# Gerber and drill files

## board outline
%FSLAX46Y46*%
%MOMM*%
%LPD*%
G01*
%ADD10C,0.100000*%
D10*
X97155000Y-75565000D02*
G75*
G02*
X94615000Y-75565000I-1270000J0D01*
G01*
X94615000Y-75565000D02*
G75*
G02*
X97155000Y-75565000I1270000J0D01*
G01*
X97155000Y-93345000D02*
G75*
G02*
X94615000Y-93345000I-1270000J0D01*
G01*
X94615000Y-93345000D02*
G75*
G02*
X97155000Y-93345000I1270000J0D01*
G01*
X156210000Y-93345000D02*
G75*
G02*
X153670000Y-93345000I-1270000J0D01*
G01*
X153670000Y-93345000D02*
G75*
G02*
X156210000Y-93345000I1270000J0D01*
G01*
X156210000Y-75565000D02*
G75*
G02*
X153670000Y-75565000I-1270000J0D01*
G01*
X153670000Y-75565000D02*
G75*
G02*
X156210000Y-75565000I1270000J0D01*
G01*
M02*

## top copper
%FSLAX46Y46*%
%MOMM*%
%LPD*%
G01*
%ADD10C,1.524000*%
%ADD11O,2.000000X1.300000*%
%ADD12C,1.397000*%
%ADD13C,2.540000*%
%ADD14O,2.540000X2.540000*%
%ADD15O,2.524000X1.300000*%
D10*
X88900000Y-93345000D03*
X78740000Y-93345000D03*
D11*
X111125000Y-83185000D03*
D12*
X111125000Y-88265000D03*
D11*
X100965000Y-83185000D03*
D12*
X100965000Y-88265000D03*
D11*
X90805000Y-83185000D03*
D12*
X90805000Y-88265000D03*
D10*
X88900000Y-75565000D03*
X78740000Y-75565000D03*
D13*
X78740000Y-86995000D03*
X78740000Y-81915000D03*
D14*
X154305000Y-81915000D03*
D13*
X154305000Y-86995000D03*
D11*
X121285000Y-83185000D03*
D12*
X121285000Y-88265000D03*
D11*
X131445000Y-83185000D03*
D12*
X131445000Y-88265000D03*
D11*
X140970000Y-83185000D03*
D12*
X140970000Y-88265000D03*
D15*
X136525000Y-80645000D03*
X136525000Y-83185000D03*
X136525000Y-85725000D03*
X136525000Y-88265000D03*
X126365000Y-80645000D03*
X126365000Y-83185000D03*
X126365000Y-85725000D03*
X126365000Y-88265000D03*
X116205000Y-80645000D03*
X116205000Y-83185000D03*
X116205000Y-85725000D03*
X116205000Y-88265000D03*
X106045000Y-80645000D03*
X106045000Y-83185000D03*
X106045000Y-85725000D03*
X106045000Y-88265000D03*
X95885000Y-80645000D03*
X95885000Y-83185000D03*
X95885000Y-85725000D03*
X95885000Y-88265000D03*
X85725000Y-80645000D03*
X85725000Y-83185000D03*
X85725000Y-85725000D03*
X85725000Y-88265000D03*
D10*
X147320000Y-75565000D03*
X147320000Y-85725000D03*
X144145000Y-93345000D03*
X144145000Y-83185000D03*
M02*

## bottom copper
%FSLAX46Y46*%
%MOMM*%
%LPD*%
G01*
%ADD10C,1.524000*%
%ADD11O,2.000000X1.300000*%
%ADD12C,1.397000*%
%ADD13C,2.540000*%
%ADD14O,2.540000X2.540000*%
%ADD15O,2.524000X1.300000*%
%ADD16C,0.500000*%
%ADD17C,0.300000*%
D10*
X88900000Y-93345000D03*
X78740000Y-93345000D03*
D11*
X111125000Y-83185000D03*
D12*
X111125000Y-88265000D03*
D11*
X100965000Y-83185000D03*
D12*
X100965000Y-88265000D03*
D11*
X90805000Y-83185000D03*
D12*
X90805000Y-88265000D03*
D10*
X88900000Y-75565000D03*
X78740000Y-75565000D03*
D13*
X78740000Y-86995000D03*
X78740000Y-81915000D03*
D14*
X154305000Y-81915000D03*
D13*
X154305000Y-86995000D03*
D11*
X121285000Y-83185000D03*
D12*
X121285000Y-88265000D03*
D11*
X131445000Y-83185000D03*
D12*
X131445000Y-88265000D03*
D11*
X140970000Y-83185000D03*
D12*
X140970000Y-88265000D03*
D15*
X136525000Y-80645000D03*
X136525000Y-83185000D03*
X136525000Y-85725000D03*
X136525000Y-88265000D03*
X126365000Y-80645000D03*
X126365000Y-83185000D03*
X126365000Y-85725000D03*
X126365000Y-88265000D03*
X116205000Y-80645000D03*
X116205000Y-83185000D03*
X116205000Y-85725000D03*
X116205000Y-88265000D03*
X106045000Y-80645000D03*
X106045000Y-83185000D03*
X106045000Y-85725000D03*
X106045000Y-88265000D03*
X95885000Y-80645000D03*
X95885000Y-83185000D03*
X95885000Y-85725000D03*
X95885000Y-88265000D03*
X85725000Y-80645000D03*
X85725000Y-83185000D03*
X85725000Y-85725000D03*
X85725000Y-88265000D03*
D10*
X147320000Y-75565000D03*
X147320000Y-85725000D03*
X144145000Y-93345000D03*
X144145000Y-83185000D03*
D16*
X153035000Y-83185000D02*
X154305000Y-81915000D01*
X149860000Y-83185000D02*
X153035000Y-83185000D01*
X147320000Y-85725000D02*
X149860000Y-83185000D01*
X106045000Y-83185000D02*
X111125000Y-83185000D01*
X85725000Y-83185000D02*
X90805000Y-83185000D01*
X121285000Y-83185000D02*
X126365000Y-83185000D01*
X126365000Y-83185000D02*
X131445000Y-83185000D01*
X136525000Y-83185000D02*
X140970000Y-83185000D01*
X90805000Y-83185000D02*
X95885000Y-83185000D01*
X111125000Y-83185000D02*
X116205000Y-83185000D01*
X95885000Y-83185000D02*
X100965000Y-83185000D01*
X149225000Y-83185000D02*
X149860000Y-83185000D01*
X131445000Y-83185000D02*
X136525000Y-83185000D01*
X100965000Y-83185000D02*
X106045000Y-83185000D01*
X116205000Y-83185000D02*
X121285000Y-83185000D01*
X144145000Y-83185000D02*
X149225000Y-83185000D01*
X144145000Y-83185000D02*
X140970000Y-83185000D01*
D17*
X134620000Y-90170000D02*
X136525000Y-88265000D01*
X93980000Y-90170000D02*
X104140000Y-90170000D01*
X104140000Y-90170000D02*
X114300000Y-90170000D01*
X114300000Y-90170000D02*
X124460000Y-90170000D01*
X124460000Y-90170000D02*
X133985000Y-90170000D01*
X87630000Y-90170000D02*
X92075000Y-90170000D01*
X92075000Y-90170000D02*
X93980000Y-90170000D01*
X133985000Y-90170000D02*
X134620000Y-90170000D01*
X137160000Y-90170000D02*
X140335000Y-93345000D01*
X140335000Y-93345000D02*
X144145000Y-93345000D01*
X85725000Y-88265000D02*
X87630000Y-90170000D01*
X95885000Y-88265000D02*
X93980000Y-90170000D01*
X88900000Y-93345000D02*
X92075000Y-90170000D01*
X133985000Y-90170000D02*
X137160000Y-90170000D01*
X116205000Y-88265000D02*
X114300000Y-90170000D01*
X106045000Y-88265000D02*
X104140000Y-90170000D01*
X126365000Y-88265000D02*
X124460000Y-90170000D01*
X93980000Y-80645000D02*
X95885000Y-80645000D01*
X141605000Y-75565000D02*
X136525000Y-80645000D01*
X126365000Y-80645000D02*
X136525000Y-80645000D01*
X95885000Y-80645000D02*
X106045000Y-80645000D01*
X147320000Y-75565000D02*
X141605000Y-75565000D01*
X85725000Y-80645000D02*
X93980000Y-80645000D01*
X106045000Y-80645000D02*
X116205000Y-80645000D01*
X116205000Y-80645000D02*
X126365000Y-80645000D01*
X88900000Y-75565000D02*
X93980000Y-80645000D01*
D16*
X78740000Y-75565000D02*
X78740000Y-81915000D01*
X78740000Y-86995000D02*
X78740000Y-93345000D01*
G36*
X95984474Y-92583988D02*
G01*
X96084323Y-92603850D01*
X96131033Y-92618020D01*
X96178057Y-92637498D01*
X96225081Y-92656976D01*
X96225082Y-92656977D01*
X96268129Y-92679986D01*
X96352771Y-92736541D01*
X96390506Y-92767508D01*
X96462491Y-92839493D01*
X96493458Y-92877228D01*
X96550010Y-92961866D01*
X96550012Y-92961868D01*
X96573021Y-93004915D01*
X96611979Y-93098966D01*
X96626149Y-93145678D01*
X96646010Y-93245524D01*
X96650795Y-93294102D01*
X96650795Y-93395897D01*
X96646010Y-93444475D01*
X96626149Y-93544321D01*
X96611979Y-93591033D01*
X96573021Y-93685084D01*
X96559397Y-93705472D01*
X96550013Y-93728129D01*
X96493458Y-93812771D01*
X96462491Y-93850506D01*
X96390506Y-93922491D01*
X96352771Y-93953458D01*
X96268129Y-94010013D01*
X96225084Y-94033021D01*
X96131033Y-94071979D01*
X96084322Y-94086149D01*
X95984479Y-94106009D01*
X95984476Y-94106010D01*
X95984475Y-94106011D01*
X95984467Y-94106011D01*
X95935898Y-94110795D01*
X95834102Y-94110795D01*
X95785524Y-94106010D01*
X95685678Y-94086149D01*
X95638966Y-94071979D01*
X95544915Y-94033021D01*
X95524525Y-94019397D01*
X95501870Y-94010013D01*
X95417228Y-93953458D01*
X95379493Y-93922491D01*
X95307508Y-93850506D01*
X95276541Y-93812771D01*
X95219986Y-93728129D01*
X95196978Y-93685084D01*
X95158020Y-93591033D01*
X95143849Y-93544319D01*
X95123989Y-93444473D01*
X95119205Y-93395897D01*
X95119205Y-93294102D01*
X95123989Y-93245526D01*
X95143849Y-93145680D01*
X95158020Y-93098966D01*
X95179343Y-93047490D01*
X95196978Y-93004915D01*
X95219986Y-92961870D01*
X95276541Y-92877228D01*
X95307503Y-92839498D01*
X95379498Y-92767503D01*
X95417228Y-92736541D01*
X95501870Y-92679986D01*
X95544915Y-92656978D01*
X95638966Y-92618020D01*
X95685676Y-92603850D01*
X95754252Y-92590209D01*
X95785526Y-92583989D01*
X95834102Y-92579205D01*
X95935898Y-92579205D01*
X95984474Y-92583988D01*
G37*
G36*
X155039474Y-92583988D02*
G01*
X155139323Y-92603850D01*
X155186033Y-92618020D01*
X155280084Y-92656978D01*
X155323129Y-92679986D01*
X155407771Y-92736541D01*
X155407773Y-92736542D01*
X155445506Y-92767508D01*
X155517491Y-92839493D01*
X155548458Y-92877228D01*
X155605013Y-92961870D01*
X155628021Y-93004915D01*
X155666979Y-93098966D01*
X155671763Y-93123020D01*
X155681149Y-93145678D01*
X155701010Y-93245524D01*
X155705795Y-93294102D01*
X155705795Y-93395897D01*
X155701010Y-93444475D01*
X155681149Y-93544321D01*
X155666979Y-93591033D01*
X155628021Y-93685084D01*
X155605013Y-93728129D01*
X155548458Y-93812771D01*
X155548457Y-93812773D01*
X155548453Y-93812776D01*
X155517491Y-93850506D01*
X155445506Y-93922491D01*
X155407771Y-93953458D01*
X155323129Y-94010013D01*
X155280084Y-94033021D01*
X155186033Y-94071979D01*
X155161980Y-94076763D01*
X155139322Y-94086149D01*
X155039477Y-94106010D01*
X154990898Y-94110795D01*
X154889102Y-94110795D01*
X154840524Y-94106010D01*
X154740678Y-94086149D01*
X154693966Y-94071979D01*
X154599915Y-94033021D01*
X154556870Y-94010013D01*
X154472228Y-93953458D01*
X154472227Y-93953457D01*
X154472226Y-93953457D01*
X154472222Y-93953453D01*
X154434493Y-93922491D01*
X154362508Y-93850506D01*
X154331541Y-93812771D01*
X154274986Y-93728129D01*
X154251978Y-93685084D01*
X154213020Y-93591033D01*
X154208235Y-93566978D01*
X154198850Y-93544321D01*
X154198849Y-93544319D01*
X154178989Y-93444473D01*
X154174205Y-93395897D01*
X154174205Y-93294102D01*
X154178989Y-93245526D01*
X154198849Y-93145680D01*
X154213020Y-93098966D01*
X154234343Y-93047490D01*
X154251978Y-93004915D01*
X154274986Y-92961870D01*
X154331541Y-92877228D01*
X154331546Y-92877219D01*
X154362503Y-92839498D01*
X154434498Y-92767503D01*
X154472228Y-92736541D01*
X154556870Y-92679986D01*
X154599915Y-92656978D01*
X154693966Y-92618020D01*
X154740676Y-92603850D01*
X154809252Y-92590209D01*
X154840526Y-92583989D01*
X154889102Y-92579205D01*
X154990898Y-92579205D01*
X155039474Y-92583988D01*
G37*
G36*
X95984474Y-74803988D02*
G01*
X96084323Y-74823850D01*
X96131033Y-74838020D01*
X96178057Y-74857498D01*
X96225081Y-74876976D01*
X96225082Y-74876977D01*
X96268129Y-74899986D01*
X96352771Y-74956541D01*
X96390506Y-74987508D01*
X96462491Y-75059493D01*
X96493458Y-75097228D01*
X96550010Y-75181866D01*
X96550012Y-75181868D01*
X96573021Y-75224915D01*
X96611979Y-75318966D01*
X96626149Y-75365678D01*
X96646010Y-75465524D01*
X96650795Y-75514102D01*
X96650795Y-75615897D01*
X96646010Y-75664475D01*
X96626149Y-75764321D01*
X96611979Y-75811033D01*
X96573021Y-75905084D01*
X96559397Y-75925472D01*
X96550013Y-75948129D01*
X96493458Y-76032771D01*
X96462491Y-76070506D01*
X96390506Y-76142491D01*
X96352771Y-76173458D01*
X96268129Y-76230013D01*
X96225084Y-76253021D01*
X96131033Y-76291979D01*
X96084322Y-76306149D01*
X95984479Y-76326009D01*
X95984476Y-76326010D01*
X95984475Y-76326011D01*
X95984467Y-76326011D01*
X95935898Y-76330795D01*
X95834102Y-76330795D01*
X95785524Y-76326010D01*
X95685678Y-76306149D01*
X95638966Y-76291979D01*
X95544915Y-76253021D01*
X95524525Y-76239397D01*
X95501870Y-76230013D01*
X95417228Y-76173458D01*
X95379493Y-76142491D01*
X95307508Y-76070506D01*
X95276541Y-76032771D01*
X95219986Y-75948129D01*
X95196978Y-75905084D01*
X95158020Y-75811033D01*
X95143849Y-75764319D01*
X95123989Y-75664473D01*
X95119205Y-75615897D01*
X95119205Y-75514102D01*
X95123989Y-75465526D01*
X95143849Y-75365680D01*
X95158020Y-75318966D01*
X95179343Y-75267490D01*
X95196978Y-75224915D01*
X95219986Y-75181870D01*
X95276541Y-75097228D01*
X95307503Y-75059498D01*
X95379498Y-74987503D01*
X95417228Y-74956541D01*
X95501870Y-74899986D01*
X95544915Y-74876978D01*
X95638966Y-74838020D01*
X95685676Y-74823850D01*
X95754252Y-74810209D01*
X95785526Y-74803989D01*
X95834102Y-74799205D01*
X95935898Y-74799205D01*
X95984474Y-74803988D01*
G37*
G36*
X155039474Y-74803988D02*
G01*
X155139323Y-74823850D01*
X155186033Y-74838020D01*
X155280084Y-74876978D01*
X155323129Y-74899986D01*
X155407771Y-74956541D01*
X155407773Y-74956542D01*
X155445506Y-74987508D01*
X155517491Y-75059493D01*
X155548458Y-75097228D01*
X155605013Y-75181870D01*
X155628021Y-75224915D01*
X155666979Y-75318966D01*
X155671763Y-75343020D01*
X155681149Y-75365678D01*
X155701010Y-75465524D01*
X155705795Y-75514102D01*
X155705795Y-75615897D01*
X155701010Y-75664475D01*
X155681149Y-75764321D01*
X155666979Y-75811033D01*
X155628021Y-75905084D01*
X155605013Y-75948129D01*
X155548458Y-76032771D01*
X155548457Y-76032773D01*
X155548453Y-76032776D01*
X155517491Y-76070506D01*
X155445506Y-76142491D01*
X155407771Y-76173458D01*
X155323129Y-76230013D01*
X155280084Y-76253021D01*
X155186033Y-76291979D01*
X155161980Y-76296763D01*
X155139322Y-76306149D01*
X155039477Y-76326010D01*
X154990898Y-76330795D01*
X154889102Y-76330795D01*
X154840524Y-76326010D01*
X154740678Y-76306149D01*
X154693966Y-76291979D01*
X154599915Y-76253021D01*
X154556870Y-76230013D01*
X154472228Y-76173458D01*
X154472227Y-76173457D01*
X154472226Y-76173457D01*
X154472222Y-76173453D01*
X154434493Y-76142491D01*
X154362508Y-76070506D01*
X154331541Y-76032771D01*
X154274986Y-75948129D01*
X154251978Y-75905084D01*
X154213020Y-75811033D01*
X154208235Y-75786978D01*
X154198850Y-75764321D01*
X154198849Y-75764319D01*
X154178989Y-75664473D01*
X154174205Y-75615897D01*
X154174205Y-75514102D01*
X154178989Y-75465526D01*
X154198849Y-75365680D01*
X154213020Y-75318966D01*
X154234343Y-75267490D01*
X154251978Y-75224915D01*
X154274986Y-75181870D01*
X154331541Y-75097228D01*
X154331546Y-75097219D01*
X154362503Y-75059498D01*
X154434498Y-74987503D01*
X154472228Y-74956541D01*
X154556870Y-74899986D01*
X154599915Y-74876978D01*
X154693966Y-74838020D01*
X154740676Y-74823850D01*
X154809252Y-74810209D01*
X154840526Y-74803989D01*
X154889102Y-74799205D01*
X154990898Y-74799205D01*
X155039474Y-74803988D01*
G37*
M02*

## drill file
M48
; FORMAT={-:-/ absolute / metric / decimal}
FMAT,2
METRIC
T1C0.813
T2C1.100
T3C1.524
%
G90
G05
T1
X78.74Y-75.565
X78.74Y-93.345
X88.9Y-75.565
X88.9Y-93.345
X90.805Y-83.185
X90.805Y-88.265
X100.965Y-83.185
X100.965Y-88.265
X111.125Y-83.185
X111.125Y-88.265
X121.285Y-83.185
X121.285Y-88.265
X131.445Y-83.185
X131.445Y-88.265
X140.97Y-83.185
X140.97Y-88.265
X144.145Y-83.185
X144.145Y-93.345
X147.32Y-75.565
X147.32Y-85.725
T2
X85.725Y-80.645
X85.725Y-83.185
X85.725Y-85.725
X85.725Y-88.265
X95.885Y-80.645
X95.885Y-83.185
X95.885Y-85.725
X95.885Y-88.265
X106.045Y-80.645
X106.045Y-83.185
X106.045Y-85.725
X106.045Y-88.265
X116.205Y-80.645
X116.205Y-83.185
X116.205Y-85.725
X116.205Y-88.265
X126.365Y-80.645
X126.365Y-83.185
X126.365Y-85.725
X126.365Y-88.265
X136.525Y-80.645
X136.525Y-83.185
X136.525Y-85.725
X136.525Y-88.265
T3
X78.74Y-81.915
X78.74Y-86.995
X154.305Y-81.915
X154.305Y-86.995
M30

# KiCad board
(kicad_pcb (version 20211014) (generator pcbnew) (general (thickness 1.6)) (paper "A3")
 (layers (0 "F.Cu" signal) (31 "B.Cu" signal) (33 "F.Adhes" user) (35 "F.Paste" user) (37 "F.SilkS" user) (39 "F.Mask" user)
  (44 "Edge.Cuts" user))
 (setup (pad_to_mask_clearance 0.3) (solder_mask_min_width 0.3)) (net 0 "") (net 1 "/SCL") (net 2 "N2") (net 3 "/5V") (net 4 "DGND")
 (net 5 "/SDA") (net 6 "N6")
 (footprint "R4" (layer "F.Cu") (at 83.82 93.345 180) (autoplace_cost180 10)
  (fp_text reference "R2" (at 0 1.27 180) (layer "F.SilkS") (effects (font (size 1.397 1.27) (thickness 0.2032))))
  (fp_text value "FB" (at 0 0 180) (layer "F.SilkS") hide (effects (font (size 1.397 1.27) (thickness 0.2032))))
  (pad "1" thru_hole circle locked (at -5.08 0 180) (size 1.524 1.524) (drill 0.8128) (layers *.Cu *.Mask "F.SilkS") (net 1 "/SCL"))
  (pad "2" thru_hole circle locked (at 5.08 0 180) (size 1.524 1.524) (drill 0.8128) (layers *.Cu *.Mask "F.SilkS") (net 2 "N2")))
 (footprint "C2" (layer "F.Cu") (at 111.125 85.725 -90)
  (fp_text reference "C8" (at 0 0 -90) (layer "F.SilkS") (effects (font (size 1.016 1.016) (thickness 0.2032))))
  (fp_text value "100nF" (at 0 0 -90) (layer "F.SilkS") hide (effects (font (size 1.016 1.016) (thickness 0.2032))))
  (pad "1" thru_hole oval locked (at -2.54 0 270) (size 1.3 2) (drill 0.8128) (layers *.Cu *.Mask "F.SilkS") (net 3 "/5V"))
  (pad "2" thru_hole circle locked (at 2.54 0 270) (size 1.397 1.397) (drill 0.8128) (layers *.Cu *.Mask "F.SilkS") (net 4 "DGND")))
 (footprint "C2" (layer "F.Cu") (at 100.965 85.725 -90)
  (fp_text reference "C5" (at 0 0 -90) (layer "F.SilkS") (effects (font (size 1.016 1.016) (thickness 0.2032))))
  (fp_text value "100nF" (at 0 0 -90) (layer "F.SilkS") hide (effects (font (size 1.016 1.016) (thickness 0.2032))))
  (pad "1" thru_hole oval locked (at -2.54 0 270) (size 1.3 2) (drill 0.8128) (layers *.Cu *.Mask "F.SilkS") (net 3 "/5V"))
  (pad "2" thru_hole circle locked (at 2.54 0 270) (size 1.397 1.397) (drill 0.8128) (layers *.Cu *.Mask "F.SilkS") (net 4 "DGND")))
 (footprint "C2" (layer "F.Cu") (at 90.805 85.725 -90)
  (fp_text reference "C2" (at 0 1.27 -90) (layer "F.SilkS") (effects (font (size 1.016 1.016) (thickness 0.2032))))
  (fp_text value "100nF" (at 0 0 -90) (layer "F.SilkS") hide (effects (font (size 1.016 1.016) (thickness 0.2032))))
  (pad "1" thru_hole oval locked (at -2.54 0 270) (size 1.3 2) (drill 0.8128) (layers *.Cu *.Mask "F.SilkS") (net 3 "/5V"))
  (pad "2" thru_hole circle locked (at 2.54 0 270) (size 1.397 1.397) (drill 0.8128) (layers *.Cu *.Mask "F.SilkS") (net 4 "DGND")))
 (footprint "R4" (layer "F.Cu") (at 83.82 75.565 180) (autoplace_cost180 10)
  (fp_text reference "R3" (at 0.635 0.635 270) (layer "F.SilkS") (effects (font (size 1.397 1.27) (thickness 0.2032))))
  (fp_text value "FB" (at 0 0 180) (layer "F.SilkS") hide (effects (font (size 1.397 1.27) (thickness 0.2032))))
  (pad "1" thru_hole circle locked (at -5.08 0 180) (size 1.524 1.524) (drill 0.8128) (layers *.Cu *.Mask "F.SilkS") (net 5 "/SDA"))
  (pad "2" thru_hole circle locked (at 5.08 0 180) (size 1.524 1.524) (drill 0.8128) (layers *.Cu *.Mask "F.SilkS") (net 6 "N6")))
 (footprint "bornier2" (layer "F.Cu") (at 78.74 84.455 90)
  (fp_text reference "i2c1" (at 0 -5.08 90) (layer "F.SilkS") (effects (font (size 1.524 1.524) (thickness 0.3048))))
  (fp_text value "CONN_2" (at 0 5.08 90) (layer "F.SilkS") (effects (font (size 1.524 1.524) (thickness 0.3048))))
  (pad "1" thru_hole circle locked (at -2.54 0 90) (size 2.54 2.54) (drill 1.524) (layers *.Cu *.Mask "F.SilkS") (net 2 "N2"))
  (pad "2" thru_hole circle locked (at 2.54 0 90) (size 2.54 2.54) (drill 1.524) (layers *.Cu *.Mask "F.SilkS") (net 6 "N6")))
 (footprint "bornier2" (layer "F.Cu") (at 154.305 84.455 -90)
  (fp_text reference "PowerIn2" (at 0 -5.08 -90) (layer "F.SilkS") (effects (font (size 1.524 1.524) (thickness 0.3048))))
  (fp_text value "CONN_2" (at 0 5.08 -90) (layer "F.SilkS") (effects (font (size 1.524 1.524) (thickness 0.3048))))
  (pad "1" thru_hole oval locked (at -2.54 0 270) (size 2.54 2.54) (drill 1.524) (layers *.Cu *.Mask "F.SilkS") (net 3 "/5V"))
  (pad "2" thru_hole circle locked (at 2.54 0 270) (size 2.54 2.54) (drill 1.524) (layers *.Cu *.Mask "F.SilkS") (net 4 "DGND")))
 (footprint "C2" (layer "F.Cu") (at 121.285 85.725 -90)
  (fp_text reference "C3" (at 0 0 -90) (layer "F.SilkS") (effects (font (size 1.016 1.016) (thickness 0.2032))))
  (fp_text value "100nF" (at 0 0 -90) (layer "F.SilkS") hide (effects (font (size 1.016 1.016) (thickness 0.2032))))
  (pad "1" thru_hole oval locked (at -2.54 0 270) (size 1.3 2) (drill 0.8128) (layers *.Cu *.Mask "F.SilkS") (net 3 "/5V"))
  (pad "2" thru_hole circle locked (at 2.54 0 270) (size 1.397 1.397) (drill 0.8128) (layers *.Cu *.Mask "F.SilkS") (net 4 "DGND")))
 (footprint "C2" (layer "F.Cu") (at 131.445 85.725 -90)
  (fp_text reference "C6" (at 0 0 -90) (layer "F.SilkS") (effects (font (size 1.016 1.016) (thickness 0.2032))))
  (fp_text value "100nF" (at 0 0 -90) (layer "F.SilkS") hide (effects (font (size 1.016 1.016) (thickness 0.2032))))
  (pad "1" thru_hole oval locked (at -2.54 0 270) (size 1.3 2) (drill 0.8128) (layers *.Cu *.Mask "F.SilkS") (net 3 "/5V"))
  (pad "2" thru_hole circle locked (at 2.54 0 270) (size 1.397 1.397) (drill 0.8128) (layers *.Cu *.Mask "F.SilkS") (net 4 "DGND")))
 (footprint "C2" (layer "F.Cu") (at 140.97 85.725 -90)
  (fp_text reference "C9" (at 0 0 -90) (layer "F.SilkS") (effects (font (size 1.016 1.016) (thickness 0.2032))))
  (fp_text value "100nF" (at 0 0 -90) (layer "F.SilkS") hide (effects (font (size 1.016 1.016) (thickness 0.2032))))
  (pad "1" thru_hole oval locked (at -2.54 0 270) (size 1.3 2) (drill 0.8128) (layers *.Cu *.Mask "F.SilkS") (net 3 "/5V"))
  (pad "2" thru_hole circle locked (at 2.54 0 270) (size 1.397 1.397) (drill 0.8128) (layers *.Cu *.Mask "F.SilkS") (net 4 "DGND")))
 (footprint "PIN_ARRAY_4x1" (layer "F.Cu") (at 136.525 84.455 -90)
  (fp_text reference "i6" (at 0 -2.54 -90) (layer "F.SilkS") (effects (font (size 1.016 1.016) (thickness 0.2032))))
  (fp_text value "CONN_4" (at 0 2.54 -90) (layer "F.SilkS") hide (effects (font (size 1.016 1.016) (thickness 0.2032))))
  (pad "1" thru_hole oval locked (at -3.81 0 270) (size 1.3 2.524) (drill 1.1) (layers *.Cu *.Mask "F.SilkS") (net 5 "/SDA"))
  (pad "2" thru_hole oval locked (at -1.27 0 270) (size 1.3 2.524) (drill 1.1) (layers *.Cu *.Mask "F.SilkS") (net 3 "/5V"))
  (pad "3" thru_hole oval locked (at 1.27 0 270) (size 1.3 2.524) (drill 1.1) (layers *.Cu *.Mask "F.SilkS") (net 4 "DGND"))
  (pad "4" thru_hole oval locked (at 3.81 0 270) (size 1.3 2.524) (drill 1.1) (layers *.Cu *.Mask "F.SilkS") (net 1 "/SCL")))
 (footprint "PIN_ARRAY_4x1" (layer "F.Cu") (at 126.365 84.455 -90)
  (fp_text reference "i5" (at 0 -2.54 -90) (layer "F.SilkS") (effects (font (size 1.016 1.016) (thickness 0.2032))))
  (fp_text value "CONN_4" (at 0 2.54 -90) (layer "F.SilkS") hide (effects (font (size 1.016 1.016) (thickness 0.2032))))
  (pad "1" thru_hole oval locked (at -3.81 0 270) (size 1.3 2.524) (drill 1.1) (layers *.Cu *.Mask "F.SilkS") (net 5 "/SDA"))
  (pad "2" thru_hole oval locked (at -1.27 0 270) (size 1.3 2.524) (drill 1.1) (layers *.Cu *.Mask "F.SilkS") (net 3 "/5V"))
  (pad "3" thru_hole oval locked (at 1.27 0 270) (size 1.3 2.524) (drill 1.1) (layers *.Cu *.Mask "F.SilkS") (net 4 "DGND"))
  (pad "4" thru_hole oval locked (at 3.81 0 270) (size 1.3 2.524) (drill 1.1) (layers *.Cu *.Mask "F.SilkS") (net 1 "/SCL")))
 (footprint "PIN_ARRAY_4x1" (layer "F.Cu") (at 116.205 84.455 -90)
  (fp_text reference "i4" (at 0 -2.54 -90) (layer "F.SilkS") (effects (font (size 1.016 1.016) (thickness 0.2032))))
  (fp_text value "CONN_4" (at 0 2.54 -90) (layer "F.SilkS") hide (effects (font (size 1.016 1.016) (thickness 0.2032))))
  (pad "1" thru_hole oval locked (at -3.81 0 270) (size 1.3 2.524) (drill 1.1) (layers *.Cu *.Mask "F.SilkS") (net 5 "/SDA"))
  (pad "2" thru_hole oval locked (at -1.27 0 270) (size 1.3 2.524) (drill 1.1) (layers *.Cu *.Mask "F.SilkS") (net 3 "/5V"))
  (pad "3" thru_hole oval locked (at 1.27 0 270) (size 1.3 2.524) (drill 1.1) (layers *.Cu *.Mask "F.SilkS") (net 4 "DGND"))
  (pad "4" thru_hole oval locked (at 3.81 0 270) (size 1.3 2.524) (drill 1.1) (layers *.Cu *.Mask "F.SilkS") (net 1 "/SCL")))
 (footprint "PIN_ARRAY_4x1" (layer "F.Cu") (at 106.045 84.455 -90)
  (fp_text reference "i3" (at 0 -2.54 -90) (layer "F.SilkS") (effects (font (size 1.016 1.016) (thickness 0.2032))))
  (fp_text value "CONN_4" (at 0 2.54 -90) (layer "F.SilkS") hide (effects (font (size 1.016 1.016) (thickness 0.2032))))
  (pad "1" thru_hole oval locked (at -3.81 0 270) (size 1.3 2.524) (drill 1.1) (layers *.Cu *.Mask "F.SilkS") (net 5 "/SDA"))
  (pad "2" thru_hole oval locked (at -1.27 0 270) (size 1.3 2.524) (drill 1.1) (layers *.Cu *.Mask "F.SilkS") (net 3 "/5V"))
  (pad "3" thru_hole oval locked (at 1.27 0 270) (size 1.3 2.524) (drill 1.1) (layers *.Cu *.Mask "F.SilkS") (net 4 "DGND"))
  (pad "4" thru_hole oval locked (at 3.81 0 270) (size 1.3 2.524) (drill 1.1) (layers *.Cu *.Mask "F.SilkS") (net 1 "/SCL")))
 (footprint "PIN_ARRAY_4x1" (layer "F.Cu") (at 95.885 84.455 -90)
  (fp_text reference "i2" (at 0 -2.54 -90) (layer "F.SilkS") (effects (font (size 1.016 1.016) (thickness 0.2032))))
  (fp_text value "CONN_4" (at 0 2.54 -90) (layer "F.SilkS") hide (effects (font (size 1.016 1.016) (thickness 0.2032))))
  (pad "1" thru_hole oval locked (at -3.81 0 270) (size 1.3 2.524) (drill 1.1) (layers *.Cu *.Mask "F.SilkS") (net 5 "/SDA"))
  (pad "2" thru_hole oval locked (at -1.27 0 270) (size 1.3 2.524) (drill 1.1) (layers *.Cu *.Mask "F.SilkS") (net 3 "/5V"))
  (pad "3" thru_hole oval locked (at 1.27 0 270) (size 1.3 2.524) (drill 1.1) (layers *.Cu *.Mask "F.SilkS") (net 4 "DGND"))
  (pad "4" thru_hole oval locked (at 3.81 0 270) (size 1.3 2.524) (drill 1.1) (layers *.Cu *.Mask "F.SilkS") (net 1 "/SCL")))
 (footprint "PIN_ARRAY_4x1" (layer "F.Cu") (at 85.725 84.455 90)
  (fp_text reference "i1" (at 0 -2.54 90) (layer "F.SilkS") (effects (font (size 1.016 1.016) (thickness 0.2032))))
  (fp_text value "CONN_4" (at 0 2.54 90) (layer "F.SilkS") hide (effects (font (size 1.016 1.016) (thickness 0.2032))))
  (pad "1" thru_hole oval locked (at 3.81 0 90) (size 1.3 2.524) (drill 1.1) (layers *.Cu *.Mask "F.SilkS") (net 5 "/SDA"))
  (pad "2" thru_hole oval locked (at 1.27 0 90) (size 1.3 2.524) (drill 1.1) (layers *.Cu *.Mask "F.SilkS") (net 3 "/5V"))
  (pad "3" thru_hole oval locked (at -1.27 0 90) (size 1.3 2.524) (drill 1.1) (layers *.Cu *.Mask "F.SilkS") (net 4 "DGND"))
  (pad "4" thru_hole oval locked (at -3.81 0 90) (size 1.3 2.524) (drill 1.1) (layers *.Cu *.Mask "F.SilkS") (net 1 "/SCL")))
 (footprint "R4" (layer "F.Cu") (at 147.32 80.645 -90) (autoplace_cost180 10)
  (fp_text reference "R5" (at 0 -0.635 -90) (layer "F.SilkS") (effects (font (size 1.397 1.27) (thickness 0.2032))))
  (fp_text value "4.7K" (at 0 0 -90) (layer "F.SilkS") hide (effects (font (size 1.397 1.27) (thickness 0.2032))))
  (pad "1" thru_hole circle locked (at -5.08 0 270) (size 1.524 1.524) (drill 0.8128) (layers *.Cu *.Mask "F.SilkS") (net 5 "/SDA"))
  (pad "2" thru_hole circle locked (at 5.08 0 270) (size 1.524 1.524) (drill 0.8128) (layers *.Cu *.Mask "F.SilkS") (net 3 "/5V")))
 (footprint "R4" (layer "F.Cu") (at 144.145 88.265 90) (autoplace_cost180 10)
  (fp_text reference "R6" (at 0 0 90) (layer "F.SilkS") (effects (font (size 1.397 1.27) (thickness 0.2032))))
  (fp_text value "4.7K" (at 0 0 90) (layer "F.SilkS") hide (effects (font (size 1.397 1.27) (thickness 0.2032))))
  (pad "1" thru_hole circle locked (at -5.08 0 90) (size 1.524 1.524) (drill 0.8128) (layers *.Cu *.Mask "F.SilkS") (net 1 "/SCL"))
  (pad "2" thru_hole circle locked (at 5.08 0 90) (size 1.524 1.524) (drill 0.8128) (layers *.Cu *.Mask "F.SilkS") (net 3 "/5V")))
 (gr_circle (center 95.885 75.565) (end 97.155 75.565) (layer "Edge.Cuts") (width 0.1) (fill none))
 (gr_circle (center 95.885 93.345) (end 97.155 93.345) (layer "Edge.Cuts") (width 0.1) (fill none))
 (gr_circle (center 154.94 93.345) (end 156.21 93.345) (layer "Edge.Cuts") (width 0.1) (fill none))
 (gr_circle (center 154.94 75.565) (end 153.67 75.565) (layer "Edge.Cuts") (width 0.1) (fill none))
 (segment (start 153.035 83.185) (end 154.305 81.915) (width 0.5) (layer "B.Cu") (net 3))
 (segment (start 149.86 83.185) (end 153.035 83.185) (width 0.5) (layer "B.Cu") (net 3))
 (segment (start 147.32 85.725) (end 149.86 83.185) (width 0.5) (layer "B.Cu") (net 3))
 (segment (start 106.045 83.185) (end 111.125 83.185) (width 0.5) (layer "B.Cu") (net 3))
 (segment (start 85.725 83.185) (end 90.805 83.185) (width 0.5) (layer "B.Cu") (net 3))
 (segment (start 121.285 83.185) (end 126.365 83.185) (width 0.5) (layer "B.Cu") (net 3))
 (segment (start 126.365 83.185) (end 131.445 83.185) (width 0.5) (layer "B.Cu") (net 3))
 (segment (start 136.525 83.185) (end 140.97 83.185) (width 0.5) (layer "B.Cu") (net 3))
 (segment (start 90.805 83.185) (end 95.885 83.185) (width 0.5) (layer "B.Cu") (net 3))
 (segment (start 111.125 83.185) (end 116.205 83.185) (width 0.5) (layer "B.Cu") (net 3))
 (segment (start 95.885 83.185) (end 100.965 83.185) (width 0.5) (layer "B.Cu") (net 3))
 (segment (start 149.225 83.185) (end 149.86 83.185) (width 0.5) (layer "B.Cu") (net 3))
 (segment (start 131.445 83.185) (end 136.525 83.185) (width 0.5) (layer "B.Cu") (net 3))
 (segment (start 100.965 83.185) (end 106.045 83.185) (width 0.5) (layer "B.Cu") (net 3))
 (segment (start 116.205 83.185) (end 121.285 83.185) (width 0.5) (layer "B.Cu") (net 3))
 (segment (start 144.145 83.185) (end 149.225 83.185) (width 0.5) (layer "B.Cu") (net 3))
 (segment (start 144.145 83.185) (end 140.97 83.185) (width 0.5) (layer "B.Cu") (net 3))
 (segment (start 134.62 90.17) (end 136.525 88.265) (width 0.3) (layer "B.Cu") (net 1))
 (segment (start 93.98 90.17) (end 104.14 90.17) (width 0.3) (layer "B.Cu") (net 1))
 (segment (start 104.14 90.17) (end 114.3 90.17) (width 0.3) (layer "B.Cu") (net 1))
 (segment (start 114.3 90.17) (end 124.46 90.17) (width 0.3) (layer "B.Cu") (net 1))
 (segment (start 124.46 90.17) (end 133.985 90.17) (width 0.3) (layer "B.Cu") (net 1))
 (segment (start 87.63 90.17) (end 92.075 90.17) (width 0.3) (layer "B.Cu") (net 1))
 (segment (start 92.075 90.17) (end 93.98 90.17) (width 0.3) (layer "B.Cu") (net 1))
 (segment (start 133.985 90.17) (end 134.62 90.17) (width 0.3) (layer "B.Cu") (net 1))
 (segment (start 137.16 90.17) (end 140.335 93.345) (width 0.3) (layer "B.Cu") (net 1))
 (segment (start 140.335 93.345) (end 144.145 93.345) (width 0.3) (layer "B.Cu") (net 1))
 (segment (start 85.725 88.265) (end 87.63 90.17) (width 0.3) (layer "B.Cu") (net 1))
 (segment (start 95.885 88.265) (end 93.98 90.17) (width 0.3) (layer "B.Cu") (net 1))
 (segment (start 88.9 93.345) (end 92.075 90.17) (width 0.3) (layer "B.Cu") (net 1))
 (segment (start 133.985 90.17) (end 137.16 90.17) (width 0.3) (layer "B.Cu") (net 1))
 (segment (start 116.205 88.265) (end 114.3 90.17) (width 0.3) (layer "B.Cu") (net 1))
 (segment (start 106.045 88.265) (end 104.14 90.17) (width 0.3) (layer "B.Cu") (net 1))
 (segment (start 126.365 88.265) (end 124.46 90.17) (width 0.3) (layer "B.Cu") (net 1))
 (segment (start 93.98 80.645) (end 95.885 80.645) (width 0.3) (layer "B.Cu") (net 5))
 (segment (start 141.605 75.565) (end 136.525 80.645) (width 0.3) (layer "B.Cu") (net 5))
 (segment (start 126.365 80.645) (end 136.525 80.645) (width 0.3) (layer "B.Cu") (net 5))
 (segment (start 95.885 80.645) (end 106.045 80.645) (width 0.3) (layer "B.Cu") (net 5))
 (segment (start 147.32 75.565) (end 141.605 75.565) (width 0.3) (layer "B.Cu") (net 5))
 (segment (start 85.725 80.645) (end 93.98 80.645) (width 0.3) (layer "B.Cu") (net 5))
 (segment (start 106.045 80.645) (end 116.205 80.645) (width 0.3) (layer "B.Cu") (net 5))
 (segment (start 116.205 80.645) (end 126.365 80.645) (width 0.3) (layer "B.Cu") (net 5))
 (segment (start 88.9 75.565) (end 93.98 80.645) (width 0.3) (layer "B.Cu") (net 5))
 (segment (start 78.74 75.565) (end 78.74 81.915) (width 0.5) (layer "B.Cu") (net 6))
 (segment (start 78.74 86.995) (end 78.74 93.345) (width 0.5) (layer "B.Cu") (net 2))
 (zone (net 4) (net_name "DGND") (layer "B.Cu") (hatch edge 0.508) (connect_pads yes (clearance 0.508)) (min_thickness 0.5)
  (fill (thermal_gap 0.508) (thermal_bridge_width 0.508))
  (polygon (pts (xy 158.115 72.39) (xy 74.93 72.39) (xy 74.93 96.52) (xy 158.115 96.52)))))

